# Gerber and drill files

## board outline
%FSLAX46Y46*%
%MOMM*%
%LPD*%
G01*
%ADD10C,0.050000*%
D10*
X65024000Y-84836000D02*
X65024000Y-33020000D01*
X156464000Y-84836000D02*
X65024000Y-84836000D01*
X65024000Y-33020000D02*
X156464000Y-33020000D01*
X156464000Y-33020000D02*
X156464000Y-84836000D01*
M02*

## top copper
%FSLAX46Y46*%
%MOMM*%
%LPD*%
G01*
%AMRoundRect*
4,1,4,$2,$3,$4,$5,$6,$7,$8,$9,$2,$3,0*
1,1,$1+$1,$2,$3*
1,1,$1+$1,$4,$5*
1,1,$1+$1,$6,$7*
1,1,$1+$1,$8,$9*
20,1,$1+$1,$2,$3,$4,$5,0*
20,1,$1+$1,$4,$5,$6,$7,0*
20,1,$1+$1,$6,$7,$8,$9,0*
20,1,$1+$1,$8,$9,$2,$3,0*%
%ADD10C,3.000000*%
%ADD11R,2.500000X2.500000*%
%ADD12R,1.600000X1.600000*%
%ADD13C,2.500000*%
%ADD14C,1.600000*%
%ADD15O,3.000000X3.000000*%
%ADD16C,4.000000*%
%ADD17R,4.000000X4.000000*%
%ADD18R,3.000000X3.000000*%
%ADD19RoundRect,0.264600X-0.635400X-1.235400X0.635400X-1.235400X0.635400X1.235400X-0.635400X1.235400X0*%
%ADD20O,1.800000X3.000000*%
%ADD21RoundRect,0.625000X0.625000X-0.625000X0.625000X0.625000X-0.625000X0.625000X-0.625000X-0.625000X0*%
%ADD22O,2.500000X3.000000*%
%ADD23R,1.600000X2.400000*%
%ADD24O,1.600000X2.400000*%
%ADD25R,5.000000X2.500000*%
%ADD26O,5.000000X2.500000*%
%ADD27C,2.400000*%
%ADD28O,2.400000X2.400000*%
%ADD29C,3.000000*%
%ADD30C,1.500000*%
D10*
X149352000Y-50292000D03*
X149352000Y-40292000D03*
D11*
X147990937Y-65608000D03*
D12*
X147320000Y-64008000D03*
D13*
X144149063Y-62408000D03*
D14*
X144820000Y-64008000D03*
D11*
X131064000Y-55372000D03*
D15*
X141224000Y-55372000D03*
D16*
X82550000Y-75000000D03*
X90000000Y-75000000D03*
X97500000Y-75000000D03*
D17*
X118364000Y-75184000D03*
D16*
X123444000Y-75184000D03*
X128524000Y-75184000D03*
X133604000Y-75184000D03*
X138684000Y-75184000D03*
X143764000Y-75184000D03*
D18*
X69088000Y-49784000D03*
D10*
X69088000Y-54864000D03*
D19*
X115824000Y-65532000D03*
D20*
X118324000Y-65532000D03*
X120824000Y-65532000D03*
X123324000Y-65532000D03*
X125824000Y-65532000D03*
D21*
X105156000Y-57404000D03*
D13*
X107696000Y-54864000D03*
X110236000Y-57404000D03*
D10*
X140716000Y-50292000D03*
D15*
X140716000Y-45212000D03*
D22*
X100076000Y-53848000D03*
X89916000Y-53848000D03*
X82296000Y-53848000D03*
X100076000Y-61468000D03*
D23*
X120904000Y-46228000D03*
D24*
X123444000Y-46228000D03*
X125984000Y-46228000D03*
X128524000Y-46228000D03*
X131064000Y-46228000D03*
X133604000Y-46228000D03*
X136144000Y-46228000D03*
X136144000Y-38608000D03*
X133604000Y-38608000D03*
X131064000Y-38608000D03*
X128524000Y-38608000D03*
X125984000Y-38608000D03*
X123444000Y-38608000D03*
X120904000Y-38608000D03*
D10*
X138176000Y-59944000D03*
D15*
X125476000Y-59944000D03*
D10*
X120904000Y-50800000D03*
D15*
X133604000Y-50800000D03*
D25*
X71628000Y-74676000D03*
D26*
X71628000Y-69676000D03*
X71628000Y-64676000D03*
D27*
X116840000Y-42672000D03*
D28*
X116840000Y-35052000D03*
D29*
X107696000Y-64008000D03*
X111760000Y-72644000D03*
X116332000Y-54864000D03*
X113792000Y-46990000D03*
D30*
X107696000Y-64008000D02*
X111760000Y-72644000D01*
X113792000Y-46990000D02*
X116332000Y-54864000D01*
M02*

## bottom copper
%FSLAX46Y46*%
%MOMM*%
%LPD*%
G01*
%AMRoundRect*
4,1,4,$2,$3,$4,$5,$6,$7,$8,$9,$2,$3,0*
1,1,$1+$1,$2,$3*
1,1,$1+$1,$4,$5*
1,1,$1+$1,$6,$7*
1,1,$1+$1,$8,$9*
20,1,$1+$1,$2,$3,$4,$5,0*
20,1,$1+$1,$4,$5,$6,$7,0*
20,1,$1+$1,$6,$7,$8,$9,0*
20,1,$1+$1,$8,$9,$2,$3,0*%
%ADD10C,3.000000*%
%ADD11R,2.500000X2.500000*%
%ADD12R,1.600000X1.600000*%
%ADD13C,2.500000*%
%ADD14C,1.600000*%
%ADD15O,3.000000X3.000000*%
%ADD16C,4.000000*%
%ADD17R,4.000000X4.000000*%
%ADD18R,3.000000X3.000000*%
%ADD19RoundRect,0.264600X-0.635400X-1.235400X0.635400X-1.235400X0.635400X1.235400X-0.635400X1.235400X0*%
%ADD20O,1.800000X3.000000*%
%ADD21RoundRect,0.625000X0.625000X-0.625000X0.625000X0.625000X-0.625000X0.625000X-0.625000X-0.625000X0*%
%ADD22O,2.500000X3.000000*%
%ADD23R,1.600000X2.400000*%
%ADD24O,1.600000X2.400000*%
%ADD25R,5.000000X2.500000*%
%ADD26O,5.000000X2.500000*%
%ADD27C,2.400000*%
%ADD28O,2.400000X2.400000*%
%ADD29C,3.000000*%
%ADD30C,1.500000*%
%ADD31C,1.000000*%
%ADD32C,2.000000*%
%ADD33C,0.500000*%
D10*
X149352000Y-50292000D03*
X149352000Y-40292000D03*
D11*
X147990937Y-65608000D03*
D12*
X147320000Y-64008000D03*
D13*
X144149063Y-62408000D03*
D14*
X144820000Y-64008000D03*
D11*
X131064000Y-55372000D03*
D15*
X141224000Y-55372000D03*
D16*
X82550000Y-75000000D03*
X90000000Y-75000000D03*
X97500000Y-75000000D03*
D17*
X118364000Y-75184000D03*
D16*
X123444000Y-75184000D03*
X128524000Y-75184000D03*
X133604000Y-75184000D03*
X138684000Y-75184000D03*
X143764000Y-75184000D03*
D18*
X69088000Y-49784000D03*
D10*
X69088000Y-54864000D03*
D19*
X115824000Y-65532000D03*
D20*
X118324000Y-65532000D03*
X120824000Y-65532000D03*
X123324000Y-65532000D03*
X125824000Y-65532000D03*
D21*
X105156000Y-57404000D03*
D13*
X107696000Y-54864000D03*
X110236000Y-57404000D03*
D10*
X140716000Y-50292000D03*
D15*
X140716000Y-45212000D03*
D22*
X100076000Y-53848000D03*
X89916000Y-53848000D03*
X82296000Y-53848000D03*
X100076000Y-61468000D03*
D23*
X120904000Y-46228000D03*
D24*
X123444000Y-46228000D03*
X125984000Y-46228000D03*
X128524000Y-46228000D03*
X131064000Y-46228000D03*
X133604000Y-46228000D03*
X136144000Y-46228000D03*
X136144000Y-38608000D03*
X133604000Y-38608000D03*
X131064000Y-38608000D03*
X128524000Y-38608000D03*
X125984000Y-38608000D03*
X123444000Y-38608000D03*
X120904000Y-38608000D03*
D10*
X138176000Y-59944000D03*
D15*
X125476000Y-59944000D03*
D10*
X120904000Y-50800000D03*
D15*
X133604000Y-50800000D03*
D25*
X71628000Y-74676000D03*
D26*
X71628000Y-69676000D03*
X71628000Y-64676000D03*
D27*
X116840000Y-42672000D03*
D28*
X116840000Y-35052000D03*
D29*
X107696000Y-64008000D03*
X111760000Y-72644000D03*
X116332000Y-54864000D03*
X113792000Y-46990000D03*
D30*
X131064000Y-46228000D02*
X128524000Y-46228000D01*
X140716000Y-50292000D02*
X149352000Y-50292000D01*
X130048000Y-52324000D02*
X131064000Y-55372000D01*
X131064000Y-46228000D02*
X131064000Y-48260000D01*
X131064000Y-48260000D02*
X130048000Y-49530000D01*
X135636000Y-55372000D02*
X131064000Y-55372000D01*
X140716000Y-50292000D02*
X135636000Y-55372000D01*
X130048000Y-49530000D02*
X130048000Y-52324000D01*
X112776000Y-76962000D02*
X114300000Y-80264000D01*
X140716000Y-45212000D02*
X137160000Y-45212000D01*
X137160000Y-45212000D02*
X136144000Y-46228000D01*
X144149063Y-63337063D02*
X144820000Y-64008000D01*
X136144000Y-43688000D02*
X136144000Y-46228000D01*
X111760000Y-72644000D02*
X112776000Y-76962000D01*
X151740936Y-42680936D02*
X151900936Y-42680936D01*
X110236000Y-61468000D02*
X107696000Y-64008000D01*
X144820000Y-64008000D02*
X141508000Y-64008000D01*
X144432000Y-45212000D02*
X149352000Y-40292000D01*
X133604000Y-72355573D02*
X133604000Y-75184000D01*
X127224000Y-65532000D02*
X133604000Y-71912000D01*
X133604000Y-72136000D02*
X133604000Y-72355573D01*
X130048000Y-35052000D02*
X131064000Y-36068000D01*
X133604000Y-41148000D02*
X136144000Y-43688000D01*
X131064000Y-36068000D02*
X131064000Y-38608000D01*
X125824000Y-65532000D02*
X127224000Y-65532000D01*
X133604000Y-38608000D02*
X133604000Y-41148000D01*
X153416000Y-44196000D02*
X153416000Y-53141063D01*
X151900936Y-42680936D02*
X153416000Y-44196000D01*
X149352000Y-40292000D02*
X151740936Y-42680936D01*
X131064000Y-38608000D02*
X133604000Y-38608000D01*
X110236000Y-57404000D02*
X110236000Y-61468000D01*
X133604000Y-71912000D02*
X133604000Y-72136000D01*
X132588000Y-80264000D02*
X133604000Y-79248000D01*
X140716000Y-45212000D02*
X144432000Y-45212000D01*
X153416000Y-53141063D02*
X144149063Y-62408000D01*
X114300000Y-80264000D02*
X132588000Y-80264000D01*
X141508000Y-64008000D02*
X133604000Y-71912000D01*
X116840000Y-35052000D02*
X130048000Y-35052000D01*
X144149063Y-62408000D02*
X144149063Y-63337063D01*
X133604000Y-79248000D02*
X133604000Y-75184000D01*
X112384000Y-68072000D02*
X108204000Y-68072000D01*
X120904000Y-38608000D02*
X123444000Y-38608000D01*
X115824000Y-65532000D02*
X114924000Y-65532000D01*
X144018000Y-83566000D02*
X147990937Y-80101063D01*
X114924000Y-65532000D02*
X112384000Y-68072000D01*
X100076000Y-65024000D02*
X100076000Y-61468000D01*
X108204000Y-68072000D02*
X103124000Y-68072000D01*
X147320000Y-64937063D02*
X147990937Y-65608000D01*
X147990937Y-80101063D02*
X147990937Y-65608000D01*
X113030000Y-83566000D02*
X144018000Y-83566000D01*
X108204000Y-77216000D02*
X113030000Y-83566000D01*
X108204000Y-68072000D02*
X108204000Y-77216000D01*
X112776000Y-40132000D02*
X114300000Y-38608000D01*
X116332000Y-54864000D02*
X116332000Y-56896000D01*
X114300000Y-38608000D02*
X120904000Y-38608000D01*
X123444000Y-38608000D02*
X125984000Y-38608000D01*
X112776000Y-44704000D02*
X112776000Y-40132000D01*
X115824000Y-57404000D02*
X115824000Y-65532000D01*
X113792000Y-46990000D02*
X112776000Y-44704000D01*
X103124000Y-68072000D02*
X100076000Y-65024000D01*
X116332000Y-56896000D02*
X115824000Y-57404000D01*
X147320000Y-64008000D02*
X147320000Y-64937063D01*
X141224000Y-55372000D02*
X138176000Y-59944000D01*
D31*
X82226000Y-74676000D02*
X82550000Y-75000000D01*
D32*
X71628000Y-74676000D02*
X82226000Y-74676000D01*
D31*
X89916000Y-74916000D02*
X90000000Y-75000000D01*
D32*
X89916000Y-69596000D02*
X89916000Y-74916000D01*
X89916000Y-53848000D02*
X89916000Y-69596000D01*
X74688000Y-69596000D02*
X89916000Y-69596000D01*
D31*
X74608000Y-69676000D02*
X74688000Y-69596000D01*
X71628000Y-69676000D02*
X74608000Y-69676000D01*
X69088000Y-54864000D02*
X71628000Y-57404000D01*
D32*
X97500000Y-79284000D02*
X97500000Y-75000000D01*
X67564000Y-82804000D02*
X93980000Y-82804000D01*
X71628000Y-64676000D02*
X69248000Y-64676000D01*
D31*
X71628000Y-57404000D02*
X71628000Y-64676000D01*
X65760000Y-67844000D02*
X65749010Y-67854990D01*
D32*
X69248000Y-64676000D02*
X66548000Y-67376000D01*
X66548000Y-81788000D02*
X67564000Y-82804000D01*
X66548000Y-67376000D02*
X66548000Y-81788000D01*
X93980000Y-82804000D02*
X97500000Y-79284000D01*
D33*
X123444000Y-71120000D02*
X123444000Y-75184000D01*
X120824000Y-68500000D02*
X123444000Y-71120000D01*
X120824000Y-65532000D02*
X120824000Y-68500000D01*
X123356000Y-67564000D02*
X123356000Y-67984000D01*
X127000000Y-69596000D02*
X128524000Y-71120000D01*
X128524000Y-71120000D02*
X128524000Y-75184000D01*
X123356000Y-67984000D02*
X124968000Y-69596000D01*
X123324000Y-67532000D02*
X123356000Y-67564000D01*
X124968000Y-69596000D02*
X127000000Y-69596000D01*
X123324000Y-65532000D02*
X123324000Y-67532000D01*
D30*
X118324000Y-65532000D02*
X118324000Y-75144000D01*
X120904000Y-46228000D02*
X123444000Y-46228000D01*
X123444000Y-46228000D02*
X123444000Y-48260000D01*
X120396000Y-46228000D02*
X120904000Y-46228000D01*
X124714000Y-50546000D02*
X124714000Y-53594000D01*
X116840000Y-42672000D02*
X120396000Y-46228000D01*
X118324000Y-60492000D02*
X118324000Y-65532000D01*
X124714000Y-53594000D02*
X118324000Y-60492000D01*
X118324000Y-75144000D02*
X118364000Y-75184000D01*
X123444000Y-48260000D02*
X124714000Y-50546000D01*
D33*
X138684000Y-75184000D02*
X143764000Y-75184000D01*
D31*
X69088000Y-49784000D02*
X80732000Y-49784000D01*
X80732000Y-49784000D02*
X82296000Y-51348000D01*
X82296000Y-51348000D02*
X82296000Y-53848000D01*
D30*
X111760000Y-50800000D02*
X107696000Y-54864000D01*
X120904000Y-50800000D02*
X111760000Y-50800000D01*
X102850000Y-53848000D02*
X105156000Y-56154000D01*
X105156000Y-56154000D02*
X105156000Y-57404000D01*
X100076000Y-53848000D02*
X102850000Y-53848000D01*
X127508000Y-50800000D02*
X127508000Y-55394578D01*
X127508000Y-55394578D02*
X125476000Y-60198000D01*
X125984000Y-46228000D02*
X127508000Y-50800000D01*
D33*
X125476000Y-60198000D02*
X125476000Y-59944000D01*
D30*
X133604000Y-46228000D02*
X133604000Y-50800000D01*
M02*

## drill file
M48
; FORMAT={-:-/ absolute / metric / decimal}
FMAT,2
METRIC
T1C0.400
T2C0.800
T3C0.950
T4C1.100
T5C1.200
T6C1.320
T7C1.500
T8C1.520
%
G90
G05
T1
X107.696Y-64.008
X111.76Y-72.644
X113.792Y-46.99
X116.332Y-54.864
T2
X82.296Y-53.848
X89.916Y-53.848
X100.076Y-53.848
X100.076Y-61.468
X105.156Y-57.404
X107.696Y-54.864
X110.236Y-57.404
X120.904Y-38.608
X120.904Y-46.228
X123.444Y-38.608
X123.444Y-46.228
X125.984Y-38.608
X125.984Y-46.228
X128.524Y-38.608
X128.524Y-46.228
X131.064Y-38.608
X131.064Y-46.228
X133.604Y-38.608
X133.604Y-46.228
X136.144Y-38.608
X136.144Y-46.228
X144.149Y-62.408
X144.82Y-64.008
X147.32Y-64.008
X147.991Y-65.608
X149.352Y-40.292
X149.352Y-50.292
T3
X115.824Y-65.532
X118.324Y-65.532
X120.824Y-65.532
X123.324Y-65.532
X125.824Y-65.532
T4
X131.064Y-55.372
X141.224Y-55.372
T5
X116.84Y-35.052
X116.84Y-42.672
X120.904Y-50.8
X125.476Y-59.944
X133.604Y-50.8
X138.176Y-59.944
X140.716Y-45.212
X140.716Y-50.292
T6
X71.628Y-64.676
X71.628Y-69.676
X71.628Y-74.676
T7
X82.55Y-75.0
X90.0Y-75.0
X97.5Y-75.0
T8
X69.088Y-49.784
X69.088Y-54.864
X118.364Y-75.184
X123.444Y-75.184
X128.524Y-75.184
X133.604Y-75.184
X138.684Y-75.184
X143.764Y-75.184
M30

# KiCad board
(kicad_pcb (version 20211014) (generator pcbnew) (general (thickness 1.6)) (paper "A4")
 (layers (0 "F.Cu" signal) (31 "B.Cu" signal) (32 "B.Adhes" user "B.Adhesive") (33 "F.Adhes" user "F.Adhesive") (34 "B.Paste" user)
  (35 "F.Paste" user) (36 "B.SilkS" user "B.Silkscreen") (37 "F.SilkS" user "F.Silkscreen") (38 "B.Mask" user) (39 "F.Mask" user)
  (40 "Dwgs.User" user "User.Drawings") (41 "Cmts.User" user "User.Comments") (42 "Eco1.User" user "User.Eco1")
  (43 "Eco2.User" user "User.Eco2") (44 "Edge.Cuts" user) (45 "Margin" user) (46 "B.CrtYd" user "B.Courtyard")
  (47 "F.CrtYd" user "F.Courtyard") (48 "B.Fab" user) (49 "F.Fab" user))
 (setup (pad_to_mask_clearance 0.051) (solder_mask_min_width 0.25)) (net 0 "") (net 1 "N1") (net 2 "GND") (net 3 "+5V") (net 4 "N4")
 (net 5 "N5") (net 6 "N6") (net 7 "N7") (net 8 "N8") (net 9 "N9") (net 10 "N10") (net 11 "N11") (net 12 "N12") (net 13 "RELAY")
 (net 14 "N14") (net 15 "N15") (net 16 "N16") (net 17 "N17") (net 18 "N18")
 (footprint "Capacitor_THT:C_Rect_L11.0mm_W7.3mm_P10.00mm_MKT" (layer "F.Cu") (at 149.352 50.292 90)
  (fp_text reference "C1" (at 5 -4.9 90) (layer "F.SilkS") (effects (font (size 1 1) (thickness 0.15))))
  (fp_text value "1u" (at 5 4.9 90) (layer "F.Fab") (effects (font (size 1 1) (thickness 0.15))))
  (pad "1" thru_hole circle locked (at 0 0 90) (size 3 3) (drill 0.8) (layers *.Cu *.Mask) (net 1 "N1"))
  (pad "2" thru_hole circle locked (at 10 0 90) (size 3 3) (drill 0.8) (layers *.Cu *.Mask) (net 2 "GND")))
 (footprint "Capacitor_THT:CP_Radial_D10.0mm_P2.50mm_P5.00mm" (layer "F.Cu") (at 147.32 64.008 180)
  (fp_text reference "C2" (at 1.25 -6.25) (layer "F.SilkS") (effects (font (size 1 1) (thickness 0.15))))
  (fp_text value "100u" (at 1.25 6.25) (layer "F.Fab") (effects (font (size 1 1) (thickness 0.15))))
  (pad "1" thru_hole rect locked (at -0.670937 -1.6 180) (size 2.5 2.5) (drill 0.8) (layers *.Cu *.Mask) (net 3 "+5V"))
  (pad "1" thru_hole rect locked (at 0 0 180) (size 1.6 1.6) (drill 0.8) (layers *.Cu *.Mask) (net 3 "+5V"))
  (pad "2" thru_hole circle locked (at 3.170937 1.6 180) (size 2.5 2.5) (drill 0.8) (layers *.Cu *.Mask) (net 2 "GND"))
  (pad "2" thru_hole circle locked (at 2.5 0 180) (size 1.6 1.6) (drill 0.8) (layers *.Cu *.Mask) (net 2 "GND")))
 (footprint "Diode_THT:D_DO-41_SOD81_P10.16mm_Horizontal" (layer "F.Cu") (at 131.064 55.372)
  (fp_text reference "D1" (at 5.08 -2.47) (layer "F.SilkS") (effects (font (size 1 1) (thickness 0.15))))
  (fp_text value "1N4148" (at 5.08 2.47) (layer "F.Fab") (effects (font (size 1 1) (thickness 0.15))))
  (pad "1" thru_hole rect locked (at 0 0) (size 2.5 2.5) (drill 1.1) (layers *.Cu *.Mask) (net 1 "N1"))
  (pad "2" thru_hole oval locked (at 10.16 0) (size 3 3) (drill 1.1) (layers *.Cu *.Mask) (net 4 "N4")))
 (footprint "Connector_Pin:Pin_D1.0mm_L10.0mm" (layer "F.Cu") (at 82.55 75)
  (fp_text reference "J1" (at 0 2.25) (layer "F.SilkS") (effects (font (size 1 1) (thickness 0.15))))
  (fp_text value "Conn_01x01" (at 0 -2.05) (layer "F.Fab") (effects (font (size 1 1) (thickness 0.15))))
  (pad "1" thru_hole circle locked (at 0 0) (size 4 4) (drill 1.5) (layers *.Cu *.Mask) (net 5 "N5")))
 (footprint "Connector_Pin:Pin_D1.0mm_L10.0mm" (layer "F.Cu") (at 90 75)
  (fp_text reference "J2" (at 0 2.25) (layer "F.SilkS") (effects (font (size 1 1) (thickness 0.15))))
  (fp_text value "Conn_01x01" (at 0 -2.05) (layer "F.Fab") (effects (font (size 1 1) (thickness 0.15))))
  (pad "1" thru_hole circle locked (at 0 0) (size 4 4) (drill 1.5) (layers *.Cu *.Mask) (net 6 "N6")))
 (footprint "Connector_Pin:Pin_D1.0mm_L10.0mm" (layer "F.Cu") (at 97.5 75)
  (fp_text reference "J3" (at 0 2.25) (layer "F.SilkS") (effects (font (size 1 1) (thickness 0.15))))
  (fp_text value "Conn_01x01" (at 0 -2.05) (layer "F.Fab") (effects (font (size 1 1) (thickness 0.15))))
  (pad "1" thru_hole circle locked (at 0 0) (size 4 4) (drill 1.5) (layers *.Cu *.Mask) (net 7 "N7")))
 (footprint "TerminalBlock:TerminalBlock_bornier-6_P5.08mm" (layer "F.Cu") (at 118.364 75.184)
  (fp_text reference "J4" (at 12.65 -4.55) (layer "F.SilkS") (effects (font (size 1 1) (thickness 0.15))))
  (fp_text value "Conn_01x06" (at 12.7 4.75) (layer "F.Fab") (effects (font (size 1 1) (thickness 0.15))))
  (pad "1" thru_hole rect locked (at 0 0) (size 4 4) (drill 1.52) (layers *.Cu *.Mask) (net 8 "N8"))
  (pad "2" thru_hole circle locked (at 5.08 0) (size 4 4) (drill 1.52) (layers *.Cu *.Mask) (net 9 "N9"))
  (pad "3" thru_hole circle locked (at 10.16 0) (size 4 4) (drill 1.52) (layers *.Cu *.Mask) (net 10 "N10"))
  (pad "4" thru_hole circle locked (at 15.24 0) (size 4 4) (drill 1.52) (layers *.Cu *.Mask) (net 2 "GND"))
  (pad "5" thru_hole circle locked (at 20.32 0) (size 4 4) (drill 1.52) (layers *.Cu *.Mask) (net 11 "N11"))
  (pad "6" thru_hole circle locked (at 25.4 0) (size 4 4) (drill 1.52) (layers *.Cu *.Mask) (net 11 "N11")))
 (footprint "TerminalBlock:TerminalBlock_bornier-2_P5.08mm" (layer "F.Cu") (at 69.088 49.784 -90)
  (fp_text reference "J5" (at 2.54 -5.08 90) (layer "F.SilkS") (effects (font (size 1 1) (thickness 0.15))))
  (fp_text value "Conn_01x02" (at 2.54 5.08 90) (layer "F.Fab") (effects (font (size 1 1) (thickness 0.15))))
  (pad "1" thru_hole rect locked (at 0 0 270) (size 3 3) (drill 1.52) (layers *.Cu *.Mask) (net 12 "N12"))
  (pad "2" thru_hole circle locked (at 5.08 0 270) (size 3 3) (drill 1.52) (layers *.Cu *.Mask) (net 7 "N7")))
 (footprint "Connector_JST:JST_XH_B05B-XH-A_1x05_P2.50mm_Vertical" (layer "F.Cu") (at 115.824 65.532)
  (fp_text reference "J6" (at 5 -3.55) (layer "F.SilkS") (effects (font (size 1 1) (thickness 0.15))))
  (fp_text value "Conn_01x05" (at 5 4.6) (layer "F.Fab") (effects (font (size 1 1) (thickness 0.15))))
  (pad "1" thru_hole roundrect locked (at 0 0) (size 1.8 3) (drill 0.95) (layers *.Cu *.Mask) (roundrect_rratio 0.147) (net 3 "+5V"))
  (pad "2" thru_hole oval locked (at 2.5 0) (size 1.8 3) (drill 0.95) (layers *.Cu *.Mask) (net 8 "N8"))
  (pad "3" thru_hole oval locked (at 5 0) (size 1.8 3) (drill 0.95) (layers *.Cu *.Mask) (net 9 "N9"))
  (pad "4" thru_hole oval locked (at 7.5 0) (size 1.8 3) (drill 0.95) (layers *.Cu *.Mask) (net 10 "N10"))
  (pad "5" thru_hole oval locked (at 10 0) (size 1.8 3) (drill 0.95) (layers *.Cu *.Mask) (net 2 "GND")))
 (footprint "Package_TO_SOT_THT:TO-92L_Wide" (layer "F.Cu") (at 105.156 57.404)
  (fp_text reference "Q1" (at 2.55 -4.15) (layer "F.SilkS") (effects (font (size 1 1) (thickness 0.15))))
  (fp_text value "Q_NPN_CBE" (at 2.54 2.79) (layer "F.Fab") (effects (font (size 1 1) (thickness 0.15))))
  (pad "1" thru_hole roundrect locked (at 0 0 90) (size 2.5 2.5) (drill 0.8) (layers *.Cu *.Mask) (roundrect_rratio 0.25) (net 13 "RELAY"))
  (pad "2" thru_hole circle locked (at 2.54 -2.54 90) (size 2.5 2.5) (drill 0.8) (layers *.Cu *.Mask) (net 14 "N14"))
  (pad "3" thru_hole circle locked (at 5.08 0 90) (size 2.5 2.5) (drill 0.8) (layers *.Cu *.Mask) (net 2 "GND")))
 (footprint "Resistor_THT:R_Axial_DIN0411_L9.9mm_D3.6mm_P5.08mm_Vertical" (layer "F.Cu") (at 140.716 50.292 90)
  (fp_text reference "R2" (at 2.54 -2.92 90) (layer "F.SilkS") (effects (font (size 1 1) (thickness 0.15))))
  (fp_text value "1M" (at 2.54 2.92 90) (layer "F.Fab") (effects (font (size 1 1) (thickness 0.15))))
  (pad "1" thru_hole circle locked (at 0 0 90) (size 3 3) (drill 1.2) (layers *.Cu *.Mask) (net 1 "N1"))
  (pad "2" thru_hole oval locked (at 5.08 0 90) (size 3 3) (drill 1.2) (layers *.Cu *.Mask) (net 2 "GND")))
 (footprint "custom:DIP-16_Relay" (layer "F.Cu") (at 100.076 53.848 -90)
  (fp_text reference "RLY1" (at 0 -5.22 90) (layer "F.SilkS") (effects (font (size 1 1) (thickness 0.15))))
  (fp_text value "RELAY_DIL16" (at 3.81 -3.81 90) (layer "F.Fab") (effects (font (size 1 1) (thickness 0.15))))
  (pad "1" thru_hole oval locked (at 0 0 270) (size 3 2.5) (drill 0.8) (layers *.Cu *.Mask "F.SilkS") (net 13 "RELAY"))
  (pad "5" thru_hole oval locked (at 0 10.16 270) (size 3 2.5) (drill 0.8) (layers *.Cu *.Mask "F.SilkS") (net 6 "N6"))
  (pad "8" thru_hole oval locked (at 0 17.78 270) (size 3 2.5) (drill 0.8) (layers *.Cu *.Mask "F.SilkS") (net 12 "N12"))
  (pad "16" thru_hole oval locked (at 7.62 0 270) (size 3 2.5) (drill 0.8) (layers *.Cu *.Mask "F.SilkS") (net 3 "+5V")))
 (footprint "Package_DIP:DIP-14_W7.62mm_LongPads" (layer "F.Cu") (at 120.904 46.228 90)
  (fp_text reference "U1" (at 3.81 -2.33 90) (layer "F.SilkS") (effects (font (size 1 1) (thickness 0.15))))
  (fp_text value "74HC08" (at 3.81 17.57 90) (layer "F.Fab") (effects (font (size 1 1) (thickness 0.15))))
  (pad "1" thru_hole rect locked (at 0 0 90) (size 2.4 1.6) (drill 0.8) (layers *.Cu *.Mask) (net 8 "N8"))
  (pad "2" thru_hole oval locked (at 0 2.54 90) (size 2.4 1.6) (drill 0.8) (layers *.Cu *.Mask) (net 8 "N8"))
  (pad "3" thru_hole oval locked (at 0 5.08 90) (size 2.4 1.6) (drill 0.8) (layers *.Cu *.Mask) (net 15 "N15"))
  (pad "4" thru_hole oval locked (at 0 7.62 90) (size 2.4 1.6) (drill 0.8) (layers *.Cu *.Mask) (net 1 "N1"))
  (pad "5" thru_hole oval locked (at 0 10.16 90) (size 2.4 1.6) (drill 0.8) (layers *.Cu *.Mask) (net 1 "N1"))
  (pad "6" thru_hole oval locked (at 0 12.7 90) (size 2.4 1.6) (drill 0.8) (layers *.Cu *.Mask) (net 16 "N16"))
  (pad "7" thru_hole oval locked (at 0 15.24 90) (size 2.4 1.6) (drill 0.8) (layers *.Cu *.Mask) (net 2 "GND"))
  (pad "8" thru_hole oval locked (at 7.62 15.24 90) (size 2.4 1.6) (drill 0.8) (layers *.Cu *.Mask) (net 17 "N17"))
  (pad "9" thru_hole oval locked (at 7.62 12.7 90) (size 2.4 1.6) (drill 0.8) (layers *.Cu *.Mask) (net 2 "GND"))
  (pad "10" thru_hole oval locked (at 7.62 10.16 90) (size 2.4 1.6) (drill 0.8) (layers *.Cu *.Mask) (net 2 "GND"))
  (pad "11" thru_hole oval locked (at 7.62 7.62 90) (size 2.4 1.6) (drill 0.8) (layers *.Cu *.Mask) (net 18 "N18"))
  (pad "12" thru_hole oval locked (at 7.62 5.08 90) (size 2.4 1.6) (drill 0.8) (layers *.Cu *.Mask) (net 3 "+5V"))
  (pad "13" thru_hole oval locked (at 7.62 2.54 90) (size 2.4 1.6) (drill 0.8) (layers *.Cu *.Mask) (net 3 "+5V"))
  (pad "14" thru_hole oval locked (at 7.62 0 90) (size 2.4 1.6) (drill 0.8) (layers *.Cu *.Mask) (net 3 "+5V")))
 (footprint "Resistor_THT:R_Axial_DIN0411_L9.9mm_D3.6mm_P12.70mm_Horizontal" (layer "F.Cu") (at 138.176 59.944 180)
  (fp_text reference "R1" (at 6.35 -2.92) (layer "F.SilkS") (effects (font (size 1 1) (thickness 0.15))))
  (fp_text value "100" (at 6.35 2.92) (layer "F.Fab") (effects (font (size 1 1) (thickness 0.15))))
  (pad "1" thru_hole circle locked (at 0 0 180) (size 3 3) (drill 1.2) (layers *.Cu *.Mask) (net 4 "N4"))
  (pad "2" thru_hole oval locked (at 12.7 0 180) (size 3 3) (drill 1.2) (layers *.Cu *.Mask) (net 15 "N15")))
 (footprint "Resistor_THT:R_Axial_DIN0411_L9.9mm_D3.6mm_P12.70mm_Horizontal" (layer "F.Cu") (at 120.904 50.8)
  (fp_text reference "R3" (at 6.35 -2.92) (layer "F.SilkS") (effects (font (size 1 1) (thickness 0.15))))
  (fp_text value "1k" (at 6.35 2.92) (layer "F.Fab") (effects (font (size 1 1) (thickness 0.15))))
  (pad "1" thru_hole circle locked (at 0 0) (size 3 3) (drill 1.2) (layers *.Cu *.Mask) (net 14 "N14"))
  (pad "2" thru_hole oval locked (at 12.7 0) (size 3 3) (drill 1.2) (layers *.Cu *.Mask) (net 16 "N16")))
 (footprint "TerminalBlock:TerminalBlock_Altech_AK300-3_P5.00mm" (layer "F.Cu") (at 71.628 74.676 90)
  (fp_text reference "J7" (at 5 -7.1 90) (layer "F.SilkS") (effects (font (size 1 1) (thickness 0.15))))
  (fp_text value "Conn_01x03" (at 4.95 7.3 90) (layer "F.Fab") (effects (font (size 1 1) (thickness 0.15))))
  (pad "1" thru_hole rect locked (at 0 0 90) (size 2.5 5) (drill 1.32) (layers *.Cu *.Mask) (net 5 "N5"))
  (pad "2" thru_hole oval locked (at 5 0 90) (size 2.5 5) (drill 1.32) (layers *.Cu *.Mask) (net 6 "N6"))
  (pad "3" thru_hole oval locked (at 10 0 90) (size 2.5 5) (drill 1.32) (layers *.Cu *.Mask) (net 7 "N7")))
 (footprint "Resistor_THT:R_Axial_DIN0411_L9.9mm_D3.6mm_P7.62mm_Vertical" (layer "F.Cu") (at 116.84 42.672 90)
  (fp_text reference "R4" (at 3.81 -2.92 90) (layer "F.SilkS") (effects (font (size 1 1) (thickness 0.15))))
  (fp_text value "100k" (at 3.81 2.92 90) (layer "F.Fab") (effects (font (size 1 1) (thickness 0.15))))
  (pad "1" thru_hole circle locked (at 0 0 90) (size 2.4 2.4) (drill 1.2) (layers *.Cu *.Mask) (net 8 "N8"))
  (pad "2" thru_hole oval locked (at 7.62 0 90) (size 2.4 2.4) (drill 1.2) (layers *.Cu *.Mask) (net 2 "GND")))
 (gr_line (start 65.024 84.836) (end 65.024 33.02) (layer "Edge.Cuts") (width 0.05))
 (gr_line (start 156.464 84.836) (end 65.024 84.836) (layer "Edge.Cuts") (width 0.05))
 (gr_line (start 65.024 33.02) (end 156.464 33.02) (layer "Edge.Cuts") (width 0.05))
 (gr_line (start 156.464 33.02) (end 156.464 84.836) (layer "Edge.Cuts") (width 0.05))
 (segment (start 131.064 46.228) (end 128.524 46.228) (width 1.5) (layer "B.Cu") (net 1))
 (segment (start 140.716 50.292) (end 149.352 50.292) (width 1.5) (layer "B.Cu") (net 1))
 (segment (start 130.048 52.324) (end 131.064 55.372) (width 1.5) (layer "B.Cu") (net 1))
 (segment (start 131.064 46.228) (end 131.064 48.26) (width 1.5) (layer "B.Cu") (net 1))
 (segment (start 131.064 48.26) (end 130.048 49.53) (width 1.5) (layer "B.Cu") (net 1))
 (segment (start 135.636 55.372) (end 131.064 55.372) (width 1.5) (layer "B.Cu") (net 1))
 (segment (start 140.716 50.292) (end 135.636 55.372) (width 1.5) (layer "B.Cu") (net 1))
 (segment (start 130.048 49.53) (end 130.048 52.324) (width 1.5) (layer "B.Cu") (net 1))
 (segment (start 107.696 64.008) (end 111.76 72.644) (width 1.5) (layer "F.Cu") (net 2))
 (via (at 107.696 64.008) (size 3) (drill 0.4) (layers "F.Cu" "B.Cu") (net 2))
 (via (at 111.76 72.644) (size 3) (drill 0.4) (layers "F.Cu" "B.Cu") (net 2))
 (segment (start 112.776 76.962) (end 114.3 80.264) (width 1.5) (layer "B.Cu") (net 2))
 (segment (start 140.716 45.212) (end 137.16 45.212) (width 1.5) (layer "B.Cu") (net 2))
 (segment (start 137.16 45.212) (end 136.144 46.228) (width 1.5) (layer "B.Cu") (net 2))
 (segment (start 144.149063 63.337063) (end 144.82 64.008) (width 1.5) (layer "B.Cu") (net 2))
 (segment (start 136.144 43.688) (end 136.144 46.228) (width 1.5) (layer "B.Cu") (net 2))
 (segment (start 111.76 72.644) (end 112.776 76.962) (width 1.5) (layer "B.Cu") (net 2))
 (segment (start 151.740936 42.680936) (end 151.900936 42.680936) (width 1.5) (layer "B.Cu") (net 2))
 (segment (start 110.236 61.468) (end 107.696 64.008) (width 1.5) (layer "B.Cu") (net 2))
 (segment (start 144.82 64.008) (end 141.508 64.008) (width 1.5) (layer "B.Cu") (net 2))
 (segment (start 144.432 45.212) (end 149.352 40.292) (width 1.5) (layer "B.Cu") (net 2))
 (segment (start 133.604 72.355573) (end 133.604 75.184) (width 1.5) (layer "B.Cu") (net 2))
 (segment (start 127.224 65.532) (end 133.604 71.912) (width 1.5) (layer "B.Cu") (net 2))
 (segment (start 133.604 72.136) (end 133.604 72.355573) (width 1.5) (layer "B.Cu") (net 2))
 (segment (start 130.048 35.052) (end 131.064 36.068) (width 1.5) (layer "B.Cu") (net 2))
 (segment (start 133.604 41.148) (end 136.144 43.688) (width 1.5) (layer "B.Cu") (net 2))
 (segment (start 131.064 36.068) (end 131.064 38.608) (width 1.5) (layer "B.Cu") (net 2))
 (segment (start 125.824 65.532) (end 127.224 65.532) (width 1.5) (layer "B.Cu") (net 2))
 (segment (start 133.604 38.608) (end 133.604 41.148) (width 1.5) (layer "B.Cu") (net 2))
 (segment (start 153.416 44.196) (end 153.416 53.141063) (width 1.5) (layer "B.Cu") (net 2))
 (segment (start 151.900936 42.680936) (end 153.416 44.196) (width 1.5) (layer "B.Cu") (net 2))
 (segment (start 149.352 40.292) (end 151.740936 42.680936) (width 1.5) (layer "B.Cu") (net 2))
 (segment (start 131.064 38.608) (end 133.604 38.608) (width 1.5) (layer "B.Cu") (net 2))
 (segment (start 110.236 57.404) (end 110.236 61.468) (width 1.5) (layer "B.Cu") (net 2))
 (segment (start 133.604 71.912) (end 133.604 72.136) (width 1.5) (layer "B.Cu") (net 2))
 (segment (start 132.588 80.264) (end 133.604 79.248) (width 1.5) (layer "B.Cu") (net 2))
 (segment (start 140.716 45.212) (end 144.432 45.212) (width 1.5) (layer "B.Cu") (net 2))
 (segment (start 153.416 53.141063) (end 144.149063 62.408) (width 1.5) (layer "B.Cu") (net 2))
 (segment (start 114.3 80.264) (end 132.588 80.264) (width 1.5) (layer "B.Cu") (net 2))
 (segment (start 141.508 64.008) (end 133.604 71.912) (width 1.5) (layer "B.Cu") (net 2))
 (segment (start 116.84 35.052) (end 130.048 35.052) (width 1.5) (layer "B.Cu") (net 2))
 (segment (start 144.149063 62.408) (end 144.149063 63.337063) (width 1.5) (layer "B.Cu") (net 2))
 (segment (start 133.604 79.248) (end 133.604 75.184) (width 1.5) (layer "B.Cu") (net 2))
 (segment (start 113.792 46.99) (end 116.332 54.864) (width 1.5) (layer "F.Cu") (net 3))
 (via (at 116.332 54.864) (size 3) (drill 0.4) (layers "F.Cu" "B.Cu") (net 3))
 (via (at 113.792 46.99) (size 3) (drill 0.4) (layers "F.Cu" "B.Cu") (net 3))
 (segment (start 112.384 68.072) (end 108.204 68.072) (width 1.5) (layer "B.Cu") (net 3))
 (segment (start 120.904 38.608) (end 123.444 38.608) (width 1.5) (layer "B.Cu") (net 3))
 (segment (start 115.824 65.532) (end 114.924 65.532) (width 1.5) (layer "B.Cu") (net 3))
 (segment (start 144.018 83.566) (end 147.990937 80.101063) (width 1.5) (layer "B.Cu") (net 3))
 (segment (start 114.924 65.532) (end 112.384 68.072) (width 1.5) (layer "B.Cu") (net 3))
 (segment (start 100.076 65.024) (end 100.076 61.468) (width 1.5) (layer "B.Cu") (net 3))
 (segment (start 108.204 68.072) (end 103.124 68.072) (width 1.5) (layer "B.Cu") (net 3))
 (segment (start 147.32 64.937063) (end 147.990937 65.608) (width 1.5) (layer "B.Cu") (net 3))
 (segment (start 147.990937 80.101063) (end 147.990937 65.608) (width 1.5) (layer "B.Cu") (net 3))
 (segment (start 113.03 83.566) (end 144.018 83.566) (width 1.5) (layer "B.Cu") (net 3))
 (segment (start 108.204 77.216) (end 113.03 83.566) (width 1.5) (layer "B.Cu") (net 3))
 (segment (start 108.204 68.072) (end 108.204 77.216) (width 1.5) (layer "B.Cu") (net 3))
 (segment (start 112.776 40.132) (end 114.3 38.608) (width 1.5) (layer "B.Cu") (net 3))
 (segment (start 116.332 54.864) (end 116.332 56.896) (width 1.5) (layer "B.Cu") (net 3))
 (segment (start 114.3 38.608) (end 120.904 38.608) (width 1.5) (layer "B.Cu") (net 3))
 (segment (start 123.444 38.608) (end 125.984 38.608) (width 1.5) (layer "B.Cu") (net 3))
 (segment (start 112.776 44.704) (end 112.776 40.132) (width 1.5) (layer "B.Cu") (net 3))
 (segment (start 115.824 57.404) (end 115.824 65.532) (width 1.5) (layer "B.Cu") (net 3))
 (segment (start 113.792 46.99) (end 112.776 44.704) (width 1.5) (layer "B.Cu") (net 3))
 (segment (start 103.124 68.072) (end 100.076 65.024) (width 1.5) (layer "B.Cu") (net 3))
 (segment (start 116.332 56.896) (end 115.824 57.404) (width 1.5) (layer "B.Cu") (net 3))
 (segment (start 147.32 64.008) (end 147.32 64.937063) (width 1.5) (layer "B.Cu") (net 3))
 (segment (start 141.224 55.372) (end 138.176 59.944) (width 1.5) (layer "B.Cu") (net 4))
 (segment (start 82.226 74.676) (end 82.55 75) (width 1) (layer "B.Cu") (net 5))
 (segment (start 71.628 74.676) (end 82.226 74.676) (width 2) (layer "B.Cu") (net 5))
 (segment (start 89.916 74.916) (end 90 75) (width 1) (layer "B.Cu") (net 6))
 (segment (start 89.916 69.596) (end 89.916 74.916) (width 2) (layer "B.Cu") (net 6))
 (segment (start 89.916 53.848) (end 89.916 69.596) (width 2) (layer "B.Cu") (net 6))
 (segment (start 74.688 69.596) (end 89.916 69.596) (width 2) (layer "B.Cu") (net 6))
 (segment (start 74.608 69.676) (end 74.688 69.596) (width 1) (layer "B.Cu") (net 6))
 (segment (start 71.628 69.676) (end 74.608 69.676) (width 1) (layer "B.Cu") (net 6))
 (segment (start 69.088 54.864) (end 71.628 57.404) (width 1) (layer "B.Cu") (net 7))
 (segment (start 97.5 79.284) (end 97.5 75) (width 2) (layer "B.Cu") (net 7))
 (segment (start 67.564 82.804) (end 93.98 82.804) (width 2) (layer "B.Cu") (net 7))
 (segment (start 71.628 64.676) (end 69.248 64.676) (width 2) (layer "B.Cu") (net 7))
 (segment (start 71.628 57.404) (end 71.628 64.676) (width 1) (layer "B.Cu") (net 7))
 (segment (start 65.76 67.844) (end 65.74901 67.85499) (width 1) (layer "B.Cu") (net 7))
 (segment (start 69.248 64.676) (end 66.548 67.376) (width 2) (layer "B.Cu") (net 7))
 (segment (start 66.548 81.788) (end 67.564 82.804) (width 2) (layer "B.Cu") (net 7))
 (segment (start 66.548 67.376) (end 66.548 81.788) (width 2) (layer "B.Cu") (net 7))
 (segment (start 93.98 82.804) (end 97.5 79.284) (width 2) (layer "B.Cu") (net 7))
 (segment (start 123.444 71.12) (end 123.444 75.184) (width 0.5) (layer "B.Cu") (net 9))
 (segment (start 120.824 68.5) (end 123.444 71.12) (width 0.5) (layer "B.Cu") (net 9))
 (segment (start 120.824 65.532) (end 120.824 68.5) (width 0.5) (layer "B.Cu") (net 9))
 (segment (start 123.356 67.564) (end 123.356 67.984) (width 0.5) (layer "B.Cu") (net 10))
 (segment (start 127 69.596) (end 128.524 71.12) (width 0.5) (layer "B.Cu") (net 10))
 (segment (start 128.524 71.12) (end 128.524 75.184) (width 0.5) (layer "B.Cu") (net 10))
 (segment (start 123.356 67.984) (end 124.968 69.596) (width 0.5) (layer "B.Cu") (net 10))
 (segment (start 123.324 67.532) (end 123.356 67.564) (width 0.5) (layer "B.Cu") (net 10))
 (segment (start 124.968 69.596) (end 127 69.596) (width 0.5) (layer "B.Cu") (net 10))
 (segment (start 123.324 65.532) (end 123.324 67.532) (width 0.5) (layer "B.Cu") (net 10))
 (segment (start 118.324 65.532) (end 118.324 75.144) (width 1.5) (layer "B.Cu") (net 8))
 (segment (start 120.904 46.228) (end 123.444 46.228) (width 1.5) (layer "B.Cu") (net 8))
 (segment (start 123.444 46.228) (end 123.444 48.26) (width 1.5) (layer "B.Cu") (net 8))
 (segment (start 120.396 46.228) (end 120.904 46.228) (width 1.5) (layer "B.Cu") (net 8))
 (segment (start 124.714 50.546) (end 124.714 53.594) (width 1.5) (layer "B.Cu") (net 8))
 (segment (start 116.84 42.672) (end 120.396 46.228) (width 1.5) (layer "B.Cu") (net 8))
 (segment (start 118.324 60.492) (end 118.324 65.532) (width 1.5) (layer "B.Cu") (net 8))
 (segment (start 124.714 53.594) (end 118.324 60.492) (width 1.5) (layer "B.Cu") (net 8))
 (segment (start 118.324 75.144) (end 118.364 75.184) (width 1.5) (layer "B.Cu") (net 8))
 (segment (start 123.444 48.26) (end 124.714 50.546) (width 1.5) (layer "B.Cu") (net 8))
 (segment (start 138.684 75.184) (end 143.764 75.184) (width 0.5) (layer "B.Cu") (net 11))
 (segment (start 69.088 49.784) (end 80.732 49.784) (width 1) (layer "B.Cu") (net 12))
 (segment (start 80.732 49.784) (end 82.296 51.348) (width 1) (layer "B.Cu") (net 12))
 (segment (start 82.296 51.348) (end 82.296 53.848) (width 1) (layer "B.Cu") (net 12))
 (segment (start 111.76 50.8) (end 107.696 54.864) (width 1.5) (layer "B.Cu") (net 14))
 (segment (start 120.904 50.8) (end 111.76 50.8) (width 1.5) (layer "B.Cu") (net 14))
 (segment (start 102.85 53.848) (end 105.156 56.154) (width 1.5) (layer "B.Cu") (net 13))
 (segment (start 105.156 56.154) (end 105.156 57.404) (width 1.5) (layer "B.Cu") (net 13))
 (segment (start 100.076 53.848) (end 102.85 53.848) (width 1.5) (layer "B.Cu") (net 13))
 (segment (start 127.508 50.8) (end 127.508 55.394578) (width 1.5) (layer "B.Cu") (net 15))
 (segment (start 127.508 55.394578) (end 125.476 60.198) (width 1.5) (layer "B.Cu") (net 15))
 (segment (start 125.984 46.228) (end 127.508 50.8) (width 1.5) (layer "B.Cu") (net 15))
 (segment (start 125.476 60.198) (end 125.476 59.944) (width 0.5) (layer "B.Cu") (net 15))
 (segment (start 133.604 46.228) (end 133.604 50.8) (width 1.5) (layer "B.Cu") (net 16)))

